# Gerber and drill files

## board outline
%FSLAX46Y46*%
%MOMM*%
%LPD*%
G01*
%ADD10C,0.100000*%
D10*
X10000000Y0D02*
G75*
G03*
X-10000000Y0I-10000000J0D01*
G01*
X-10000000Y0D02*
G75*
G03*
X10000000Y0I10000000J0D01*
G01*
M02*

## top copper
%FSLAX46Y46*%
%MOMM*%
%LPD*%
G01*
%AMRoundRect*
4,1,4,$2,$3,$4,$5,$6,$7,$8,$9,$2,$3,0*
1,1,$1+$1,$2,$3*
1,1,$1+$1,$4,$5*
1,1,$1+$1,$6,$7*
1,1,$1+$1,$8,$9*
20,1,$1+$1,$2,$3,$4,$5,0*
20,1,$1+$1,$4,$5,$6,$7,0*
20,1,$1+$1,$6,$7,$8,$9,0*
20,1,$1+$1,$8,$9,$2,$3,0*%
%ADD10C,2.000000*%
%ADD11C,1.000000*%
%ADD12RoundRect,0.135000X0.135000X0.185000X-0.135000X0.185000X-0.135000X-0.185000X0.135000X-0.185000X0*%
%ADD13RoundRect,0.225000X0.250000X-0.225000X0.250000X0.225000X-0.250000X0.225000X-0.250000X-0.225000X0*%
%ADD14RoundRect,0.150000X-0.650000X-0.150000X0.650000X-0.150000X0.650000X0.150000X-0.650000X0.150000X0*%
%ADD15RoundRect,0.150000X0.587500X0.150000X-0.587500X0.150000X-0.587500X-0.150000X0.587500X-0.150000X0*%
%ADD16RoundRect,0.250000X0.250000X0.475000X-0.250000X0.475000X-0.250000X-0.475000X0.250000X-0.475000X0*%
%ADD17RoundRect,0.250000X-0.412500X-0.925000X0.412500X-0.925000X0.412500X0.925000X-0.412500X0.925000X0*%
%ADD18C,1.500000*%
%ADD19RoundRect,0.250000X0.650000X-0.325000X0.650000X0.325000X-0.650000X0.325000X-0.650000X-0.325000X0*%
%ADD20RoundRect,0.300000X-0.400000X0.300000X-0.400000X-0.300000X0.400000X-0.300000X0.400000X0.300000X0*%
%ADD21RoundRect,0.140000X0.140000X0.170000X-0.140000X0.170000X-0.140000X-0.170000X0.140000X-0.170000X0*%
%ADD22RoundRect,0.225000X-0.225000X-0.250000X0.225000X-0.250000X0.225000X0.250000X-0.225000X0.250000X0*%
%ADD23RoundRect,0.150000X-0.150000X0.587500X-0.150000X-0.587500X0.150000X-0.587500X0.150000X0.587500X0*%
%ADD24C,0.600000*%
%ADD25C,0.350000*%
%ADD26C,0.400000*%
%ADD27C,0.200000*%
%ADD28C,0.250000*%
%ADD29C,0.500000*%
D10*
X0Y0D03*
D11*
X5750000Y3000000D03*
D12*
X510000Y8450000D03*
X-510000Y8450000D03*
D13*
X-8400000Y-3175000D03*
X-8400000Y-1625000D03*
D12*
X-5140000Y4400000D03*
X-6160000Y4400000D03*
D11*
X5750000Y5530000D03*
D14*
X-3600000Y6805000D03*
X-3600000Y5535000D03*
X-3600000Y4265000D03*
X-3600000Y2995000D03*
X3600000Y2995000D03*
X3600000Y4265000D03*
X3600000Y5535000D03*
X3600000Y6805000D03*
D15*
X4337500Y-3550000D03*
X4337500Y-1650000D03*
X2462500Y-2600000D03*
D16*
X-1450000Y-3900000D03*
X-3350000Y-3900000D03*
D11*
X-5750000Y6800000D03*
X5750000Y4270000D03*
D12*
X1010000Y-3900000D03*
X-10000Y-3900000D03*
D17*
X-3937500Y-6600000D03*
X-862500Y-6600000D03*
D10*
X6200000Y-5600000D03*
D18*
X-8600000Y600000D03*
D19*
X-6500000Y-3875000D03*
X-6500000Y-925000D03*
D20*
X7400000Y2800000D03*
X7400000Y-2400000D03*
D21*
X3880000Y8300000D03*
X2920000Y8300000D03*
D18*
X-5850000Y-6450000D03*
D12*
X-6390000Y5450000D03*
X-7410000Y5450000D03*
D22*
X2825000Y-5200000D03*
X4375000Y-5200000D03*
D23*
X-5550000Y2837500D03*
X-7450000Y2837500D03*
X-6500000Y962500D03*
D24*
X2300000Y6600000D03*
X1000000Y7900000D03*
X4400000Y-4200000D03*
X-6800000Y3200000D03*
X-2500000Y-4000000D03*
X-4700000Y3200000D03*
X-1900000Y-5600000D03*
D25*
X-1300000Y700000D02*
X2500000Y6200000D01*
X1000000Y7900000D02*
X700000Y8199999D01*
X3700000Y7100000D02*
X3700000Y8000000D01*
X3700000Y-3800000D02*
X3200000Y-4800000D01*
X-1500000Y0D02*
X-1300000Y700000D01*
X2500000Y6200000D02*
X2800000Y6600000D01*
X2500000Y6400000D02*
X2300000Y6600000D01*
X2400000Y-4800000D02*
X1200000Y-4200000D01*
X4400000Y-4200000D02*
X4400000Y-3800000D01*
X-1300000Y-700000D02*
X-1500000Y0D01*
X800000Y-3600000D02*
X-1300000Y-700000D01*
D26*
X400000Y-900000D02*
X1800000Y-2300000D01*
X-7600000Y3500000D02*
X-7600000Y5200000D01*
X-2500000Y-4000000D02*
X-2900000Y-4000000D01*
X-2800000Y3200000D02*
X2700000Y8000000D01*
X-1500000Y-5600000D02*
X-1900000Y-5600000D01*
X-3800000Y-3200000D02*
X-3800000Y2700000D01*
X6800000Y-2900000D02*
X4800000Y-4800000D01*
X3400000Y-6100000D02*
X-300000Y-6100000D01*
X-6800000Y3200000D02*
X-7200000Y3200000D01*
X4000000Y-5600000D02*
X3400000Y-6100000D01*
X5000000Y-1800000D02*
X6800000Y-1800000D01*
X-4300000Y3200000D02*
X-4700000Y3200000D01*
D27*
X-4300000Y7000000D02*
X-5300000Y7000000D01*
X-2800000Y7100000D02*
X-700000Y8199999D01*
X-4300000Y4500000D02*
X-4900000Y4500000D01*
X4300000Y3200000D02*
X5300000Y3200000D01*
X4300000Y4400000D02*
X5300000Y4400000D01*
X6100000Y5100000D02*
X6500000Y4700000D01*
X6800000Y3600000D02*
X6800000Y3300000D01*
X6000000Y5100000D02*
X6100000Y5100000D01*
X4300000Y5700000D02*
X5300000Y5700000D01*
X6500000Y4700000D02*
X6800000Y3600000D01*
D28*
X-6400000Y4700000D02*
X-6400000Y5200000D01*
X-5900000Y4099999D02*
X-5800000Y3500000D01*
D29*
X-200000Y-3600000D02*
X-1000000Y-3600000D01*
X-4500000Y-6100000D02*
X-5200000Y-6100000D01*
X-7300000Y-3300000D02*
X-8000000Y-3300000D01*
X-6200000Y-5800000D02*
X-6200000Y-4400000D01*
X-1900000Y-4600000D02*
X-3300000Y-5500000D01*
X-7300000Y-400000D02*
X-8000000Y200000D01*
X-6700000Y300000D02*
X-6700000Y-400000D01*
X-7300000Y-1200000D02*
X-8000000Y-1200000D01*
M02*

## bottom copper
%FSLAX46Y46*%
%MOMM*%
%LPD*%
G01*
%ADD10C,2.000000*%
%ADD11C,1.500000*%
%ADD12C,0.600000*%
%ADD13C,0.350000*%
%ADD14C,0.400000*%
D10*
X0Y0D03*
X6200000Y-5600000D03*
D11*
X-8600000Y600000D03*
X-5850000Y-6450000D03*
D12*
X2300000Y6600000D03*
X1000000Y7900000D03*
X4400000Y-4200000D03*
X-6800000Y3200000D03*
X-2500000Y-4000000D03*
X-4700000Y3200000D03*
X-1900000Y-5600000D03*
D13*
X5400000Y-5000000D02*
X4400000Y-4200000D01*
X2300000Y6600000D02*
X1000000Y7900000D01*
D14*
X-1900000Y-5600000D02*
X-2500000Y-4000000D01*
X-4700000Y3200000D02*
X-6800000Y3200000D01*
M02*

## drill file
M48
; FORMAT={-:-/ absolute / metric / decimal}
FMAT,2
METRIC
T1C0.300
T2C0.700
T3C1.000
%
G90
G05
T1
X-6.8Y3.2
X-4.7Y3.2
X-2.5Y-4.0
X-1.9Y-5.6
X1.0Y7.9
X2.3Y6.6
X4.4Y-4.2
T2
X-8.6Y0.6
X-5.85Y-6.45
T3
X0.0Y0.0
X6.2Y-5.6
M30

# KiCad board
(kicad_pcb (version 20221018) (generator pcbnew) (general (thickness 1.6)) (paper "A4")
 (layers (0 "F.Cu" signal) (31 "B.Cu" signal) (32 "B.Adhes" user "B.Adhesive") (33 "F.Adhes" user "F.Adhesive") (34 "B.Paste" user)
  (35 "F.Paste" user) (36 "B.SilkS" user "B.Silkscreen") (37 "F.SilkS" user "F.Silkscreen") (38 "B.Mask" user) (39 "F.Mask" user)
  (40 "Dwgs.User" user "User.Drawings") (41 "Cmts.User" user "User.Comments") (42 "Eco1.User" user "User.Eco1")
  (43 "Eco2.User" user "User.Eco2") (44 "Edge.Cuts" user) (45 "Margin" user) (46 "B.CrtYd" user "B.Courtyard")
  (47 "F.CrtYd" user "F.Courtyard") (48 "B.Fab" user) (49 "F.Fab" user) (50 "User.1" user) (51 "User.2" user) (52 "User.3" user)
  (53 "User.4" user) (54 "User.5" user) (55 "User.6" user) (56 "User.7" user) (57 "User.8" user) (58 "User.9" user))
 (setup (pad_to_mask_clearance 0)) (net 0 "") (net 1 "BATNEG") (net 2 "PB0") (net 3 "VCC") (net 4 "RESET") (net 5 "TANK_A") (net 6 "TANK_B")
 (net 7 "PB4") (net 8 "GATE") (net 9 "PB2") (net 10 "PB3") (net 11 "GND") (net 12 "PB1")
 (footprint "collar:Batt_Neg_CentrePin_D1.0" (layer "F.Cu") (at 0 0)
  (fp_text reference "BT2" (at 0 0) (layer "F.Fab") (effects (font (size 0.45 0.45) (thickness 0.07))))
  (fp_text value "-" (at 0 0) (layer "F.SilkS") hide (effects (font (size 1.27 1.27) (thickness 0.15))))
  (pad "1" thru_hole circle (at 0 0) (size 2 2) (drill 1) (layers "*.Cu" "*.Mask") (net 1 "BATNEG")))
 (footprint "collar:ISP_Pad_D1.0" (layer "F.Cu") (at 5.75 -3)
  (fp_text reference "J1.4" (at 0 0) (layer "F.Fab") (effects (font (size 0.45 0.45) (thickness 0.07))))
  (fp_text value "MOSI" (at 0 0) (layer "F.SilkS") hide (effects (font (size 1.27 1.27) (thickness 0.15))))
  (pad "1" smd circle (at 0 0) (size 1 1) (layers "F.Cu" "F.Mask") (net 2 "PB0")))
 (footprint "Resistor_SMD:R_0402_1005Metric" (layer "F.Cu") (at 0 -8.45 180)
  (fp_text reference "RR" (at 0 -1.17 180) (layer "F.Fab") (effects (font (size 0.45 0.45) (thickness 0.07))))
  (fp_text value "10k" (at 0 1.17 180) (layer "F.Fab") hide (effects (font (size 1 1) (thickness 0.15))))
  (pad "1" smd roundrect (at -0.51 0 180) (size 0.54 0.64) (layers "F.Cu" "F.Paste" "F.Mask") (roundrect_rratio 0.25) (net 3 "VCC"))
  (pad "2" smd roundrect (at 0.51 0 180) (size 0.54 0.64) (layers "F.Cu" "F.Paste" "F.Mask") (roundrect_rratio 0.25) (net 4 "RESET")))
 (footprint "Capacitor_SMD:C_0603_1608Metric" (layer "F.Cu") (at -8.4 2.4 90)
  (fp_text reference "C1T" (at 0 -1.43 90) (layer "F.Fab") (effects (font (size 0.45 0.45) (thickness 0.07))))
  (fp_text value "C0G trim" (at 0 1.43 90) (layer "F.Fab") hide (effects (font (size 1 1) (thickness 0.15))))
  (pad "1" smd roundrect (at -0.775 0 90) (size 0.9 0.95) (layers "F.Cu" "F.Paste" "F.Mask") (roundrect_rratio 0.25) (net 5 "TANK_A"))
  (pad "2" smd roundrect (at 0.775 0 90) (size 0.9 0.95) (layers "F.Cu" "F.Paste" "F.Mask") (roundrect_rratio 0.25) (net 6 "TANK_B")))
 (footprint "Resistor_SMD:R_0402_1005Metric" (layer "F.Cu") (at -5.65 -4.4 180)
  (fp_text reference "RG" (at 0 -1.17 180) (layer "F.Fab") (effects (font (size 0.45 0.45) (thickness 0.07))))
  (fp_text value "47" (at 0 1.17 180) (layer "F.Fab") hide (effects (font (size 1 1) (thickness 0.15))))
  (pad "1" smd roundrect (at -0.51 0 180) (size 0.54 0.64) (layers "F.Cu" "F.Paste" "F.Mask") (roundrect_rratio 0.25) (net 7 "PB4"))
  (pad "2" smd roundrect (at 0.51 0 180) (size 0.54 0.64) (layers "F.Cu" "F.Paste" "F.Mask") (roundrect_rratio 0.25) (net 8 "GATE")))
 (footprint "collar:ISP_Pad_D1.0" (layer "F.Cu") (at 5.75 -5.53)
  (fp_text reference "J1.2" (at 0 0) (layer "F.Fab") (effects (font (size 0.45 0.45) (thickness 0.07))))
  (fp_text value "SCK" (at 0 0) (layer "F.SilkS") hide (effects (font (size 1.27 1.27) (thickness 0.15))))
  (pad "1" smd circle (at 0 0) (size 1 1) (layers "F.Cu" "F.Mask") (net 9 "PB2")))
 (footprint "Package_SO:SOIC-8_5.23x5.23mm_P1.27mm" (layer "F.Cu") (at 0 -4.9)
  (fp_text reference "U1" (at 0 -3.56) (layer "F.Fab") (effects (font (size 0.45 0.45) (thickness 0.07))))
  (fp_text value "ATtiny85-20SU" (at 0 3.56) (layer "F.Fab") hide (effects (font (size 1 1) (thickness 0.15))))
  (pad "1" smd roundrect (at -3.6 -1.905) (size 1.6 0.6) (layers "F.Cu" "F.Paste" "F.Mask") (roundrect_rratio 0.25) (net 4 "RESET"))
  (pad "2" smd roundrect (at -3.6 -0.635) (size 1.6 0.6) (layers "F.Cu" "F.Paste" "F.Mask") (roundrect_rratio 0.25) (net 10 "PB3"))
  (pad "3" smd roundrect (at -3.6 0.635) (size 1.6 0.6) (layers "F.Cu" "F.Paste" "F.Mask") (roundrect_rratio 0.25) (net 7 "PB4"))
  (pad "4" smd roundrect (at -3.6 1.905) (size 1.6 0.6) (layers "F.Cu" "F.Paste" "F.Mask") (roundrect_rratio 0.25) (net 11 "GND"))
  (pad "5" smd roundrect (at 3.6 1.905) (size 1.6 0.6) (layers "F.Cu" "F.Paste" "F.Mask") (roundrect_rratio 0.25) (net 2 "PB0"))
  (pad "6" smd roundrect (at 3.6 0.635) (size 1.6 0.6) (layers "F.Cu" "F.Paste" "F.Mask") (roundrect_rratio 0.25) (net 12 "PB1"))
  (pad "7" smd roundrect (at 3.6 -0.635) (size 1.6 0.6) (layers "F.Cu" "F.Paste" "F.Mask") (roundrect_rratio 0.25) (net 9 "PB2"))
  (pad "8" smd roundrect (at 3.6 -1.905) (size 1.6 0.6) (layers "F.Cu" "F.Paste" "F.Mask") (roundrect_rratio 0.25) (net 3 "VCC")))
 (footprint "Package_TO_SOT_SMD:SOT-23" (layer "F.Cu") (at 3.4 2.6 180)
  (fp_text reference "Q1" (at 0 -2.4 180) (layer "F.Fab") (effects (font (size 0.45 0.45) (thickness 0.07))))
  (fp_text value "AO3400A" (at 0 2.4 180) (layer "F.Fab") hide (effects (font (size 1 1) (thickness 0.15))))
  (pad "1" smd roundrect (at -0.9375 -0.95 180) (size 1.475 0.6) (layers "F.Cu" "F.Paste" "F.Mask") (roundrect_rratio 0.25) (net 3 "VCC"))
  (pad "2" smd roundrect (at -0.9375 0.95 180) (size 1.475 0.6) (layers "F.Cu" "F.Paste" "F.Mask") (roundrect_rratio 0.25) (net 11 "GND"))
  (pad "3" smd roundrect (at 0.9375 0 180) (size 1.475 0.6) (layers "F.Cu" "F.Paste" "F.Mask") (roundrect_rratio 0.25) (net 1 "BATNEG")))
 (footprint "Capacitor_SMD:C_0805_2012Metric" (layer "F.Cu") (at -2.4 3.9 180)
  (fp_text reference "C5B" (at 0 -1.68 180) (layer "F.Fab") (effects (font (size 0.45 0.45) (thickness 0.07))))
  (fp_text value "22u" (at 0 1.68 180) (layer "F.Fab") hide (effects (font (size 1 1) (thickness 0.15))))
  (pad "1" smd roundrect (at -0.95 0 180) (size 1 1.45) (layers "F.Cu" "F.Paste" "F.Mask") (roundrect_rratio 0.25) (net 5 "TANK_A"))
  (pad "2" smd roundrect (at 0.95 0 180) (size 1 1.45) (layers "F.Cu" "F.Paste" "F.Mask") (roundrect_rratio 0.25) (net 11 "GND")))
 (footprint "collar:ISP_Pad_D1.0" (layer "F.Cu") (at -5.75 -6.8)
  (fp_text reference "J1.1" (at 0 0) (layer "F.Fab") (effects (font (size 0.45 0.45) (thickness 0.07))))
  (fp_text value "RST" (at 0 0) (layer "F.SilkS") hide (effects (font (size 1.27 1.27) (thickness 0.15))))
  (pad "1" smd circle (at 0 0) (size 1 1) (layers "F.Cu" "F.Mask") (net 4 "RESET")))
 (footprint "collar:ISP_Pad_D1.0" (layer "F.Cu") (at 5.75 -4.27)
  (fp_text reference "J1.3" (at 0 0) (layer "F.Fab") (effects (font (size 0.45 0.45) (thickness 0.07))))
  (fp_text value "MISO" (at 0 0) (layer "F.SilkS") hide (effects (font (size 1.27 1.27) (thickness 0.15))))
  (pad "1" smd circle (at 0 0) (size 1 1) (layers "F.Cu" "F.Mask") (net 12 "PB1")))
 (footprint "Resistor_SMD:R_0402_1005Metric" (layer "F.Cu") (at 0.5 3.9 180)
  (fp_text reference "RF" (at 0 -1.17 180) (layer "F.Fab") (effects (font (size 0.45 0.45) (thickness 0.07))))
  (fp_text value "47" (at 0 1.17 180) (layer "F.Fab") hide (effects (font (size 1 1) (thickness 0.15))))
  (pad "1" smd roundrect (at -0.51 0 180) (size 0.54 0.64) (layers "F.Cu" "F.Paste" "F.Mask") (roundrect_rratio 0.25) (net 3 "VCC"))
  (pad "2" smd roundrect (at 0.51 0 180) (size 0.54 0.64) (layers "F.Cu" "F.Paste" "F.Mask") (roundrect_rratio 0.25) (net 5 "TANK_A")))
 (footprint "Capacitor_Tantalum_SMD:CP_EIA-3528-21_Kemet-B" (layer "F.Cu") (at -2.4 6.6)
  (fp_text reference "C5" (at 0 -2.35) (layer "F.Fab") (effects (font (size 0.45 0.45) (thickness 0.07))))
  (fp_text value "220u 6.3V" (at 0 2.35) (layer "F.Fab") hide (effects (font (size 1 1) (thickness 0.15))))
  (pad "1" smd roundrect (at -1.5375 0) (size 1.325 2.35) (layers "F.Cu" "F.Paste" "F.Mask") (roundrect_rratio 0.188679) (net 5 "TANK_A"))
  (pad "2" smd roundrect (at 1.5375 0) (size 1.325 2.35) (layers "F.Cu" "F.Paste" "F.Mask") (roundrect_rratio 0.188679) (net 11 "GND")))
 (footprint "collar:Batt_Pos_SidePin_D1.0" (layer "F.Cu") (at 6.2 5.6)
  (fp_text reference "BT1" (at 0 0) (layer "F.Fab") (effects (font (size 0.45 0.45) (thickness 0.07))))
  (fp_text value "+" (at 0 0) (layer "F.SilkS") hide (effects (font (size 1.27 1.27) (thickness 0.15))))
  (pad "1" thru_hole circle (at 0 0) (size 2 2) (drill 1) (layers "*.Cu" "*.Mask") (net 3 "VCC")))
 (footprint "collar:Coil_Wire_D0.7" (layer "F.Cu") (at -8.6 -0.6)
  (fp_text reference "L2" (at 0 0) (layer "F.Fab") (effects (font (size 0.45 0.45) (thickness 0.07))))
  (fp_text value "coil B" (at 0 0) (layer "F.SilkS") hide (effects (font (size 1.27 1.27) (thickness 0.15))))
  (pad "1" thru_hole circle (at 0 0) (size 1.5 1.5) (drill 0.7) (layers "*.Cu" "*.Mask") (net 6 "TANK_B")))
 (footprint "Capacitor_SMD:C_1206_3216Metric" (layer "F.Cu") (at -6.5 2.4 90)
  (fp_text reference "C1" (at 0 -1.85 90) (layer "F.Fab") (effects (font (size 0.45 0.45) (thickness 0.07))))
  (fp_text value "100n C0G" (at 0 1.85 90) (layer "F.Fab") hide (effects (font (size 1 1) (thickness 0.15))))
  (pad "1" smd roundrect (at -1.475 0 90) (size 1.15 1.8) (layers "F.Cu" "F.Paste" "F.Mask") (roundrect_rratio 0.217391) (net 5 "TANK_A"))
  (pad "2" smd roundrect (at 1.475 0 90) (size 1.15 1.8) (layers "F.Cu" "F.Paste" "F.Mask") (roundrect_rratio 0.217391) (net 6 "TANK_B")))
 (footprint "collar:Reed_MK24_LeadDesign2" (layer "F.Cu") (at 7.4 -0.2 -90)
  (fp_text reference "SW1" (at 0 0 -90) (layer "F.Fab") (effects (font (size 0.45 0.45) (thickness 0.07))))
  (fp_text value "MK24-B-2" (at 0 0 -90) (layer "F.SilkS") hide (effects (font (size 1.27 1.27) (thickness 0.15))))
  (pad "1" smd roundrect (at -2.6 0 270) (size 1.2 1.4) (layers "F.Cu" "F.Paste" "F.Mask") (roundrect_rratio 0.25) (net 9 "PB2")
   (thermal_bridge_angle 45))
  (pad "2" smd roundrect (at 2.6 0 270) (size 1.2 1.4) (layers "F.Cu" "F.Paste" "F.Mask") (roundrect_rratio 0.25) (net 11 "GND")
   (thermal_bridge_angle 45)))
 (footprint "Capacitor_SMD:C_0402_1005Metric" (layer "F.Cu") (at 3.4 -8.3 180)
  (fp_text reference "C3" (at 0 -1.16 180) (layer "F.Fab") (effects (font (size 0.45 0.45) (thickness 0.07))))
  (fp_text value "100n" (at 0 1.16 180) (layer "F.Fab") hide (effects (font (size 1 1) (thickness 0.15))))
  (pad "1" smd roundrect (at -0.48 0 180) (size 0.56 0.62) (layers "F.Cu" "F.Paste" "F.Mask") (roundrect_rratio 0.25) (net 3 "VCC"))
  (pad "2" smd roundrect (at 0.48 0 180) (size 0.56 0.62) (layers "F.Cu" "F.Paste" "F.Mask") (roundrect_rratio 0.25) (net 11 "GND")))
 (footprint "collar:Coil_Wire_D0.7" (layer "F.Cu") (at -5.85 6.45)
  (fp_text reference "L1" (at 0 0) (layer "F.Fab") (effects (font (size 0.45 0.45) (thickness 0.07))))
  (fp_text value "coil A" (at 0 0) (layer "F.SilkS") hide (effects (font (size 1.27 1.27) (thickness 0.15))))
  (pad "1" thru_hole circle (at 0 0) (size 1.5 1.5) (drill 0.7) (layers "*.Cu" "*.Mask") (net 5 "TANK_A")))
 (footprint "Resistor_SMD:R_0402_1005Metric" (layer "F.Cu") (at -6.9 -5.45 180)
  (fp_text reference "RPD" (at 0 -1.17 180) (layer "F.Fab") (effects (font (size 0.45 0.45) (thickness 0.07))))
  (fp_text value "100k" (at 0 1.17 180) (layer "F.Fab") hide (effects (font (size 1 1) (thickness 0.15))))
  (pad "1" smd roundrect (at -0.51 0 180) (size 0.54 0.64) (layers "F.Cu" "F.Paste" "F.Mask") (roundrect_rratio 0.25) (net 8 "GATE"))
  (pad "2" smd roundrect (at 0.51 0 180) (size 0.54 0.64) (layers "F.Cu" "F.Paste" "F.Mask") (roundrect_rratio 0.25) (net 11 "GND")))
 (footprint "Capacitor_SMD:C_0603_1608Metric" (layer "F.Cu") (at 3.6 5.2)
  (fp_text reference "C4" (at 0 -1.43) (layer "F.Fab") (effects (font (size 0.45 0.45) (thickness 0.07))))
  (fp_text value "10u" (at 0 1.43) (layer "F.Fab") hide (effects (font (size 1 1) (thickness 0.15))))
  (pad "1" smd roundrect (at -0.775 0) (size 0.9 0.95) (layers "F.Cu" "F.Paste" "F.Mask") (roundrect_rratio 0.25) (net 3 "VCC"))
  (pad "2" smd roundrect (at 0.775 0) (size 0.9 0.95) (layers "F.Cu" "F.Paste" "F.Mask") (roundrect_rratio 0.25) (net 11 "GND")))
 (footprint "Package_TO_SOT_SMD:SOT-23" (layer "F.Cu") (at -6.5 -1.9 -90)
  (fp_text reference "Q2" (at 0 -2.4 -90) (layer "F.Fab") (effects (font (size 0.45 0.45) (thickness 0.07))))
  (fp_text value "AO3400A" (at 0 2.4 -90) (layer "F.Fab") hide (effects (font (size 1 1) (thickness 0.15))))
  (pad "1" smd roundrect (at -0.9375 -0.95 270) (size 1.475 0.6) (layers "F.Cu" "F.Paste" "F.Mask") (roundrect_rratio 0.25) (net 8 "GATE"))
  (pad "2" smd roundrect (at -0.9375 0.95 270) (size 1.475 0.6) (layers "F.Cu" "F.Paste" "F.Mask") (roundrect_rratio 0.25) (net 11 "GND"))
  (pad "3" smd roundrect (at 0.9375 0 270) (size 1.475 0.6) (layers "F.Cu" "F.Paste" "F.Mask") (roundrect_rratio 0.25) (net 6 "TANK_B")))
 (gr_circle (center 0 0) (end 10 0) (stroke (width 0.1) (type default)) (fill none) (layer "Edge.Cuts"))
 (segment (start -1.3 -0.7) (end 2.5 -6.2) (width 0.35) (layer "F.Cu") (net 3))
 (segment (start 1 -7.9) (end 0.7 -8.199999) (width 0.35) (layer "F.Cu") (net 3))
 (segment (start 3.7 -7.1) (end 3.7 -8) (width 0.35) (layer "F.Cu") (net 3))
 (segment (start 3.7 3.8) (end 3.2 4.8) (width 0.35) (layer "F.Cu") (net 3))
 (segment (start -1.5 0) (end -1.3 -0.7) (width 0.35) (layer "F.Cu") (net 3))
 (segment (start 2.5 -6.2) (end 2.8 -6.6) (width 0.35) (layer "F.Cu") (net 3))
 (segment (start 2.5 -6.4) (end 2.3 -6.6) (width 0.35) (layer "F.Cu") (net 3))
 (segment (start 2.4 4.8) (end 1.2 4.2) (width 0.35) (layer "F.Cu") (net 3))
 (segment (start 4.4 4.2) (end 4.4 3.8) (width 0.35) (layer "F.Cu") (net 3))
 (segment (start -1.3 0.7) (end -1.5 0) (width 0.35) (layer "F.Cu") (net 3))
 (segment (start 0.8 3.6) (end -1.3 0.7) (width 0.35) (layer "F.Cu") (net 3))
 (via (at 2.3 -6.6) (size 0.6) (drill 0.3) (layers "F.Cu" "B.Cu") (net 3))
 (via (at 1 -7.9) (size 0.6) (drill 0.3) (layers "F.Cu" "B.Cu") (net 3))
 (via (at 4.4 4.2) (size 0.6) (drill 0.3) (layers "F.Cu" "B.Cu") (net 3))
 (segment (start 5.4 5) (end 4.4 4.2) (width 0.35) (layer "B.Cu") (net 3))
 (segment (start 2.3 -6.6) (end 1 -7.9) (width 0.35) (layer "B.Cu") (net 3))
 (segment (start 0.4 0.9) (end 1.8 2.3) (width 0.4) (layer "F.Cu") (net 1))
 (segment (start -7.6 -3.5) (end -7.6 -5.2) (width 0.4) (layer "F.Cu") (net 11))
 (segment (start -2.5 4) (end -2.9 4) (width 0.4) (layer "F.Cu") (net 11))
 (segment (start -2.8 -3.2) (end 2.7 -8) (width 0.4) (layer "F.Cu") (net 11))
 (segment (start -1.5 5.6) (end -1.9 5.6) (width 0.4) (layer "F.Cu") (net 11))
 (segment (start -3.8 3.2) (end -3.8 -2.7) (width 0.4) (layer "F.Cu") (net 11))
 (segment (start 6.8 2.9) (end 4.8 4.8) (width 0.4) (layer "F.Cu") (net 11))
 (segment (start 3.4 6.1) (end -0.3 6.1) (width 0.4) (layer "F.Cu") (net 11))
 (segment (start -6.8 -3.2) (end -7.2 -3.2) (width 0.4) (layer "F.Cu") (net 11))
 (segment (start 4 5.6) (end 3.4 6.1) (width 0.4) (layer "F.Cu") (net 11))
 (segment (start 5 1.8) (end 6.8 1.8) (width 0.4) (layer "F.Cu") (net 11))
 (segment (start -4.3 -3.2) (end -4.7 -3.2) (width 0.4) (layer "F.Cu") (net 11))
 (via (at -6.8 -3.2) (size 0.6) (drill 0.3) (layers "F.Cu" "B.Cu") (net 11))
 (via (at -2.5 4) (size 0.6) (drill 0.3) (layers "F.Cu" "B.Cu") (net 11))
 (via (at -4.7 -3.2) (size 0.6) (drill 0.3) (layers "F.Cu" "B.Cu") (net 11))
 (via (at -1.9 5.6) (size 0.6) (drill 0.3) (layers "F.Cu" "B.Cu") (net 11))
 (segment (start -1.9 5.6) (end -2.5 4) (width 0.4) (layer "B.Cu") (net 11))
 (segment (start -4.7 -3.2) (end -6.8 -3.2) (width 0.4) (layer "B.Cu") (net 11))
 (segment (start -4.3 -7) (end -5.3 -7) (width 0.2) (layer "F.Cu") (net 4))
 (segment (start -2.8 -7.1) (end -0.7 -8.199999) (width 0.2) (layer "F.Cu") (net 4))
 (segment (start -4.3 -4.5) (end -4.9 -4.5) (width 0.2) (layer "F.Cu") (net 7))
 (segment (start 4.3 -3.2) (end 5.3 -3.2) (width 0.2) (layer "F.Cu") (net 2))
 (segment (start 4.3 -4.4) (end 5.3 -4.4) (width 0.2) (layer "F.Cu") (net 12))
 (segment (start 6.1 -5.1) (end 6.5 -4.7) (width 0.2) (layer "F.Cu") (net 9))
 (segment (start 6.8 -3.6) (end 6.8 -3.3) (width 0.2) (layer "F.Cu") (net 9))
 (segment (start 6 -5.1) (end 6.1 -5.1) (width 0.2) (layer "F.Cu") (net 9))
 (segment (start 4.3 -5.7) (end 5.3 -5.7) (width 0.2) (layer "F.Cu") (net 9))
 (segment (start 6.5 -4.7) (end 6.8 -3.6) (width 0.2) (layer "F.Cu") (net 9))
 (segment (start -6.4 -4.7) (end -6.4 -5.2) (width 0.25) (layer "F.Cu") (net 8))
 (segment (start -5.9 -4.099999) (end -5.8 -3.5) (width 0.25) (layer "F.Cu") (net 8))
 (segment (start -0.2 3.6) (end -1 3.6) (width 0.5) (layer "F.Cu") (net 5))
 (segment (start -4.5 6.1) (end -5.2 6.1) (width 0.5) (layer "F.Cu") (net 5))
 (segment (start -7.3 3.3) (end -8 3.3) (width 0.5) (layer "F.Cu") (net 5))
 (segment (start -6.2 5.8) (end -6.2 4.4) (width 0.5) (layer "F.Cu") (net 5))
 (segment (start -1.9 4.6) (end -3.3 5.5) (width 0.5) (layer "F.Cu") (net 5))
 (segment (start -7.3 0.4) (end -8 -0.2) (width 0.5) (layer "F.Cu") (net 6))
 (segment (start -6.7 -0.3) (end -6.7 0.4) (width 0.5) (layer "F.Cu") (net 6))
 (segment (start -7.3 1.2) (end -8 1.2) (width 0.5) (layer "F.Cu") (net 6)))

